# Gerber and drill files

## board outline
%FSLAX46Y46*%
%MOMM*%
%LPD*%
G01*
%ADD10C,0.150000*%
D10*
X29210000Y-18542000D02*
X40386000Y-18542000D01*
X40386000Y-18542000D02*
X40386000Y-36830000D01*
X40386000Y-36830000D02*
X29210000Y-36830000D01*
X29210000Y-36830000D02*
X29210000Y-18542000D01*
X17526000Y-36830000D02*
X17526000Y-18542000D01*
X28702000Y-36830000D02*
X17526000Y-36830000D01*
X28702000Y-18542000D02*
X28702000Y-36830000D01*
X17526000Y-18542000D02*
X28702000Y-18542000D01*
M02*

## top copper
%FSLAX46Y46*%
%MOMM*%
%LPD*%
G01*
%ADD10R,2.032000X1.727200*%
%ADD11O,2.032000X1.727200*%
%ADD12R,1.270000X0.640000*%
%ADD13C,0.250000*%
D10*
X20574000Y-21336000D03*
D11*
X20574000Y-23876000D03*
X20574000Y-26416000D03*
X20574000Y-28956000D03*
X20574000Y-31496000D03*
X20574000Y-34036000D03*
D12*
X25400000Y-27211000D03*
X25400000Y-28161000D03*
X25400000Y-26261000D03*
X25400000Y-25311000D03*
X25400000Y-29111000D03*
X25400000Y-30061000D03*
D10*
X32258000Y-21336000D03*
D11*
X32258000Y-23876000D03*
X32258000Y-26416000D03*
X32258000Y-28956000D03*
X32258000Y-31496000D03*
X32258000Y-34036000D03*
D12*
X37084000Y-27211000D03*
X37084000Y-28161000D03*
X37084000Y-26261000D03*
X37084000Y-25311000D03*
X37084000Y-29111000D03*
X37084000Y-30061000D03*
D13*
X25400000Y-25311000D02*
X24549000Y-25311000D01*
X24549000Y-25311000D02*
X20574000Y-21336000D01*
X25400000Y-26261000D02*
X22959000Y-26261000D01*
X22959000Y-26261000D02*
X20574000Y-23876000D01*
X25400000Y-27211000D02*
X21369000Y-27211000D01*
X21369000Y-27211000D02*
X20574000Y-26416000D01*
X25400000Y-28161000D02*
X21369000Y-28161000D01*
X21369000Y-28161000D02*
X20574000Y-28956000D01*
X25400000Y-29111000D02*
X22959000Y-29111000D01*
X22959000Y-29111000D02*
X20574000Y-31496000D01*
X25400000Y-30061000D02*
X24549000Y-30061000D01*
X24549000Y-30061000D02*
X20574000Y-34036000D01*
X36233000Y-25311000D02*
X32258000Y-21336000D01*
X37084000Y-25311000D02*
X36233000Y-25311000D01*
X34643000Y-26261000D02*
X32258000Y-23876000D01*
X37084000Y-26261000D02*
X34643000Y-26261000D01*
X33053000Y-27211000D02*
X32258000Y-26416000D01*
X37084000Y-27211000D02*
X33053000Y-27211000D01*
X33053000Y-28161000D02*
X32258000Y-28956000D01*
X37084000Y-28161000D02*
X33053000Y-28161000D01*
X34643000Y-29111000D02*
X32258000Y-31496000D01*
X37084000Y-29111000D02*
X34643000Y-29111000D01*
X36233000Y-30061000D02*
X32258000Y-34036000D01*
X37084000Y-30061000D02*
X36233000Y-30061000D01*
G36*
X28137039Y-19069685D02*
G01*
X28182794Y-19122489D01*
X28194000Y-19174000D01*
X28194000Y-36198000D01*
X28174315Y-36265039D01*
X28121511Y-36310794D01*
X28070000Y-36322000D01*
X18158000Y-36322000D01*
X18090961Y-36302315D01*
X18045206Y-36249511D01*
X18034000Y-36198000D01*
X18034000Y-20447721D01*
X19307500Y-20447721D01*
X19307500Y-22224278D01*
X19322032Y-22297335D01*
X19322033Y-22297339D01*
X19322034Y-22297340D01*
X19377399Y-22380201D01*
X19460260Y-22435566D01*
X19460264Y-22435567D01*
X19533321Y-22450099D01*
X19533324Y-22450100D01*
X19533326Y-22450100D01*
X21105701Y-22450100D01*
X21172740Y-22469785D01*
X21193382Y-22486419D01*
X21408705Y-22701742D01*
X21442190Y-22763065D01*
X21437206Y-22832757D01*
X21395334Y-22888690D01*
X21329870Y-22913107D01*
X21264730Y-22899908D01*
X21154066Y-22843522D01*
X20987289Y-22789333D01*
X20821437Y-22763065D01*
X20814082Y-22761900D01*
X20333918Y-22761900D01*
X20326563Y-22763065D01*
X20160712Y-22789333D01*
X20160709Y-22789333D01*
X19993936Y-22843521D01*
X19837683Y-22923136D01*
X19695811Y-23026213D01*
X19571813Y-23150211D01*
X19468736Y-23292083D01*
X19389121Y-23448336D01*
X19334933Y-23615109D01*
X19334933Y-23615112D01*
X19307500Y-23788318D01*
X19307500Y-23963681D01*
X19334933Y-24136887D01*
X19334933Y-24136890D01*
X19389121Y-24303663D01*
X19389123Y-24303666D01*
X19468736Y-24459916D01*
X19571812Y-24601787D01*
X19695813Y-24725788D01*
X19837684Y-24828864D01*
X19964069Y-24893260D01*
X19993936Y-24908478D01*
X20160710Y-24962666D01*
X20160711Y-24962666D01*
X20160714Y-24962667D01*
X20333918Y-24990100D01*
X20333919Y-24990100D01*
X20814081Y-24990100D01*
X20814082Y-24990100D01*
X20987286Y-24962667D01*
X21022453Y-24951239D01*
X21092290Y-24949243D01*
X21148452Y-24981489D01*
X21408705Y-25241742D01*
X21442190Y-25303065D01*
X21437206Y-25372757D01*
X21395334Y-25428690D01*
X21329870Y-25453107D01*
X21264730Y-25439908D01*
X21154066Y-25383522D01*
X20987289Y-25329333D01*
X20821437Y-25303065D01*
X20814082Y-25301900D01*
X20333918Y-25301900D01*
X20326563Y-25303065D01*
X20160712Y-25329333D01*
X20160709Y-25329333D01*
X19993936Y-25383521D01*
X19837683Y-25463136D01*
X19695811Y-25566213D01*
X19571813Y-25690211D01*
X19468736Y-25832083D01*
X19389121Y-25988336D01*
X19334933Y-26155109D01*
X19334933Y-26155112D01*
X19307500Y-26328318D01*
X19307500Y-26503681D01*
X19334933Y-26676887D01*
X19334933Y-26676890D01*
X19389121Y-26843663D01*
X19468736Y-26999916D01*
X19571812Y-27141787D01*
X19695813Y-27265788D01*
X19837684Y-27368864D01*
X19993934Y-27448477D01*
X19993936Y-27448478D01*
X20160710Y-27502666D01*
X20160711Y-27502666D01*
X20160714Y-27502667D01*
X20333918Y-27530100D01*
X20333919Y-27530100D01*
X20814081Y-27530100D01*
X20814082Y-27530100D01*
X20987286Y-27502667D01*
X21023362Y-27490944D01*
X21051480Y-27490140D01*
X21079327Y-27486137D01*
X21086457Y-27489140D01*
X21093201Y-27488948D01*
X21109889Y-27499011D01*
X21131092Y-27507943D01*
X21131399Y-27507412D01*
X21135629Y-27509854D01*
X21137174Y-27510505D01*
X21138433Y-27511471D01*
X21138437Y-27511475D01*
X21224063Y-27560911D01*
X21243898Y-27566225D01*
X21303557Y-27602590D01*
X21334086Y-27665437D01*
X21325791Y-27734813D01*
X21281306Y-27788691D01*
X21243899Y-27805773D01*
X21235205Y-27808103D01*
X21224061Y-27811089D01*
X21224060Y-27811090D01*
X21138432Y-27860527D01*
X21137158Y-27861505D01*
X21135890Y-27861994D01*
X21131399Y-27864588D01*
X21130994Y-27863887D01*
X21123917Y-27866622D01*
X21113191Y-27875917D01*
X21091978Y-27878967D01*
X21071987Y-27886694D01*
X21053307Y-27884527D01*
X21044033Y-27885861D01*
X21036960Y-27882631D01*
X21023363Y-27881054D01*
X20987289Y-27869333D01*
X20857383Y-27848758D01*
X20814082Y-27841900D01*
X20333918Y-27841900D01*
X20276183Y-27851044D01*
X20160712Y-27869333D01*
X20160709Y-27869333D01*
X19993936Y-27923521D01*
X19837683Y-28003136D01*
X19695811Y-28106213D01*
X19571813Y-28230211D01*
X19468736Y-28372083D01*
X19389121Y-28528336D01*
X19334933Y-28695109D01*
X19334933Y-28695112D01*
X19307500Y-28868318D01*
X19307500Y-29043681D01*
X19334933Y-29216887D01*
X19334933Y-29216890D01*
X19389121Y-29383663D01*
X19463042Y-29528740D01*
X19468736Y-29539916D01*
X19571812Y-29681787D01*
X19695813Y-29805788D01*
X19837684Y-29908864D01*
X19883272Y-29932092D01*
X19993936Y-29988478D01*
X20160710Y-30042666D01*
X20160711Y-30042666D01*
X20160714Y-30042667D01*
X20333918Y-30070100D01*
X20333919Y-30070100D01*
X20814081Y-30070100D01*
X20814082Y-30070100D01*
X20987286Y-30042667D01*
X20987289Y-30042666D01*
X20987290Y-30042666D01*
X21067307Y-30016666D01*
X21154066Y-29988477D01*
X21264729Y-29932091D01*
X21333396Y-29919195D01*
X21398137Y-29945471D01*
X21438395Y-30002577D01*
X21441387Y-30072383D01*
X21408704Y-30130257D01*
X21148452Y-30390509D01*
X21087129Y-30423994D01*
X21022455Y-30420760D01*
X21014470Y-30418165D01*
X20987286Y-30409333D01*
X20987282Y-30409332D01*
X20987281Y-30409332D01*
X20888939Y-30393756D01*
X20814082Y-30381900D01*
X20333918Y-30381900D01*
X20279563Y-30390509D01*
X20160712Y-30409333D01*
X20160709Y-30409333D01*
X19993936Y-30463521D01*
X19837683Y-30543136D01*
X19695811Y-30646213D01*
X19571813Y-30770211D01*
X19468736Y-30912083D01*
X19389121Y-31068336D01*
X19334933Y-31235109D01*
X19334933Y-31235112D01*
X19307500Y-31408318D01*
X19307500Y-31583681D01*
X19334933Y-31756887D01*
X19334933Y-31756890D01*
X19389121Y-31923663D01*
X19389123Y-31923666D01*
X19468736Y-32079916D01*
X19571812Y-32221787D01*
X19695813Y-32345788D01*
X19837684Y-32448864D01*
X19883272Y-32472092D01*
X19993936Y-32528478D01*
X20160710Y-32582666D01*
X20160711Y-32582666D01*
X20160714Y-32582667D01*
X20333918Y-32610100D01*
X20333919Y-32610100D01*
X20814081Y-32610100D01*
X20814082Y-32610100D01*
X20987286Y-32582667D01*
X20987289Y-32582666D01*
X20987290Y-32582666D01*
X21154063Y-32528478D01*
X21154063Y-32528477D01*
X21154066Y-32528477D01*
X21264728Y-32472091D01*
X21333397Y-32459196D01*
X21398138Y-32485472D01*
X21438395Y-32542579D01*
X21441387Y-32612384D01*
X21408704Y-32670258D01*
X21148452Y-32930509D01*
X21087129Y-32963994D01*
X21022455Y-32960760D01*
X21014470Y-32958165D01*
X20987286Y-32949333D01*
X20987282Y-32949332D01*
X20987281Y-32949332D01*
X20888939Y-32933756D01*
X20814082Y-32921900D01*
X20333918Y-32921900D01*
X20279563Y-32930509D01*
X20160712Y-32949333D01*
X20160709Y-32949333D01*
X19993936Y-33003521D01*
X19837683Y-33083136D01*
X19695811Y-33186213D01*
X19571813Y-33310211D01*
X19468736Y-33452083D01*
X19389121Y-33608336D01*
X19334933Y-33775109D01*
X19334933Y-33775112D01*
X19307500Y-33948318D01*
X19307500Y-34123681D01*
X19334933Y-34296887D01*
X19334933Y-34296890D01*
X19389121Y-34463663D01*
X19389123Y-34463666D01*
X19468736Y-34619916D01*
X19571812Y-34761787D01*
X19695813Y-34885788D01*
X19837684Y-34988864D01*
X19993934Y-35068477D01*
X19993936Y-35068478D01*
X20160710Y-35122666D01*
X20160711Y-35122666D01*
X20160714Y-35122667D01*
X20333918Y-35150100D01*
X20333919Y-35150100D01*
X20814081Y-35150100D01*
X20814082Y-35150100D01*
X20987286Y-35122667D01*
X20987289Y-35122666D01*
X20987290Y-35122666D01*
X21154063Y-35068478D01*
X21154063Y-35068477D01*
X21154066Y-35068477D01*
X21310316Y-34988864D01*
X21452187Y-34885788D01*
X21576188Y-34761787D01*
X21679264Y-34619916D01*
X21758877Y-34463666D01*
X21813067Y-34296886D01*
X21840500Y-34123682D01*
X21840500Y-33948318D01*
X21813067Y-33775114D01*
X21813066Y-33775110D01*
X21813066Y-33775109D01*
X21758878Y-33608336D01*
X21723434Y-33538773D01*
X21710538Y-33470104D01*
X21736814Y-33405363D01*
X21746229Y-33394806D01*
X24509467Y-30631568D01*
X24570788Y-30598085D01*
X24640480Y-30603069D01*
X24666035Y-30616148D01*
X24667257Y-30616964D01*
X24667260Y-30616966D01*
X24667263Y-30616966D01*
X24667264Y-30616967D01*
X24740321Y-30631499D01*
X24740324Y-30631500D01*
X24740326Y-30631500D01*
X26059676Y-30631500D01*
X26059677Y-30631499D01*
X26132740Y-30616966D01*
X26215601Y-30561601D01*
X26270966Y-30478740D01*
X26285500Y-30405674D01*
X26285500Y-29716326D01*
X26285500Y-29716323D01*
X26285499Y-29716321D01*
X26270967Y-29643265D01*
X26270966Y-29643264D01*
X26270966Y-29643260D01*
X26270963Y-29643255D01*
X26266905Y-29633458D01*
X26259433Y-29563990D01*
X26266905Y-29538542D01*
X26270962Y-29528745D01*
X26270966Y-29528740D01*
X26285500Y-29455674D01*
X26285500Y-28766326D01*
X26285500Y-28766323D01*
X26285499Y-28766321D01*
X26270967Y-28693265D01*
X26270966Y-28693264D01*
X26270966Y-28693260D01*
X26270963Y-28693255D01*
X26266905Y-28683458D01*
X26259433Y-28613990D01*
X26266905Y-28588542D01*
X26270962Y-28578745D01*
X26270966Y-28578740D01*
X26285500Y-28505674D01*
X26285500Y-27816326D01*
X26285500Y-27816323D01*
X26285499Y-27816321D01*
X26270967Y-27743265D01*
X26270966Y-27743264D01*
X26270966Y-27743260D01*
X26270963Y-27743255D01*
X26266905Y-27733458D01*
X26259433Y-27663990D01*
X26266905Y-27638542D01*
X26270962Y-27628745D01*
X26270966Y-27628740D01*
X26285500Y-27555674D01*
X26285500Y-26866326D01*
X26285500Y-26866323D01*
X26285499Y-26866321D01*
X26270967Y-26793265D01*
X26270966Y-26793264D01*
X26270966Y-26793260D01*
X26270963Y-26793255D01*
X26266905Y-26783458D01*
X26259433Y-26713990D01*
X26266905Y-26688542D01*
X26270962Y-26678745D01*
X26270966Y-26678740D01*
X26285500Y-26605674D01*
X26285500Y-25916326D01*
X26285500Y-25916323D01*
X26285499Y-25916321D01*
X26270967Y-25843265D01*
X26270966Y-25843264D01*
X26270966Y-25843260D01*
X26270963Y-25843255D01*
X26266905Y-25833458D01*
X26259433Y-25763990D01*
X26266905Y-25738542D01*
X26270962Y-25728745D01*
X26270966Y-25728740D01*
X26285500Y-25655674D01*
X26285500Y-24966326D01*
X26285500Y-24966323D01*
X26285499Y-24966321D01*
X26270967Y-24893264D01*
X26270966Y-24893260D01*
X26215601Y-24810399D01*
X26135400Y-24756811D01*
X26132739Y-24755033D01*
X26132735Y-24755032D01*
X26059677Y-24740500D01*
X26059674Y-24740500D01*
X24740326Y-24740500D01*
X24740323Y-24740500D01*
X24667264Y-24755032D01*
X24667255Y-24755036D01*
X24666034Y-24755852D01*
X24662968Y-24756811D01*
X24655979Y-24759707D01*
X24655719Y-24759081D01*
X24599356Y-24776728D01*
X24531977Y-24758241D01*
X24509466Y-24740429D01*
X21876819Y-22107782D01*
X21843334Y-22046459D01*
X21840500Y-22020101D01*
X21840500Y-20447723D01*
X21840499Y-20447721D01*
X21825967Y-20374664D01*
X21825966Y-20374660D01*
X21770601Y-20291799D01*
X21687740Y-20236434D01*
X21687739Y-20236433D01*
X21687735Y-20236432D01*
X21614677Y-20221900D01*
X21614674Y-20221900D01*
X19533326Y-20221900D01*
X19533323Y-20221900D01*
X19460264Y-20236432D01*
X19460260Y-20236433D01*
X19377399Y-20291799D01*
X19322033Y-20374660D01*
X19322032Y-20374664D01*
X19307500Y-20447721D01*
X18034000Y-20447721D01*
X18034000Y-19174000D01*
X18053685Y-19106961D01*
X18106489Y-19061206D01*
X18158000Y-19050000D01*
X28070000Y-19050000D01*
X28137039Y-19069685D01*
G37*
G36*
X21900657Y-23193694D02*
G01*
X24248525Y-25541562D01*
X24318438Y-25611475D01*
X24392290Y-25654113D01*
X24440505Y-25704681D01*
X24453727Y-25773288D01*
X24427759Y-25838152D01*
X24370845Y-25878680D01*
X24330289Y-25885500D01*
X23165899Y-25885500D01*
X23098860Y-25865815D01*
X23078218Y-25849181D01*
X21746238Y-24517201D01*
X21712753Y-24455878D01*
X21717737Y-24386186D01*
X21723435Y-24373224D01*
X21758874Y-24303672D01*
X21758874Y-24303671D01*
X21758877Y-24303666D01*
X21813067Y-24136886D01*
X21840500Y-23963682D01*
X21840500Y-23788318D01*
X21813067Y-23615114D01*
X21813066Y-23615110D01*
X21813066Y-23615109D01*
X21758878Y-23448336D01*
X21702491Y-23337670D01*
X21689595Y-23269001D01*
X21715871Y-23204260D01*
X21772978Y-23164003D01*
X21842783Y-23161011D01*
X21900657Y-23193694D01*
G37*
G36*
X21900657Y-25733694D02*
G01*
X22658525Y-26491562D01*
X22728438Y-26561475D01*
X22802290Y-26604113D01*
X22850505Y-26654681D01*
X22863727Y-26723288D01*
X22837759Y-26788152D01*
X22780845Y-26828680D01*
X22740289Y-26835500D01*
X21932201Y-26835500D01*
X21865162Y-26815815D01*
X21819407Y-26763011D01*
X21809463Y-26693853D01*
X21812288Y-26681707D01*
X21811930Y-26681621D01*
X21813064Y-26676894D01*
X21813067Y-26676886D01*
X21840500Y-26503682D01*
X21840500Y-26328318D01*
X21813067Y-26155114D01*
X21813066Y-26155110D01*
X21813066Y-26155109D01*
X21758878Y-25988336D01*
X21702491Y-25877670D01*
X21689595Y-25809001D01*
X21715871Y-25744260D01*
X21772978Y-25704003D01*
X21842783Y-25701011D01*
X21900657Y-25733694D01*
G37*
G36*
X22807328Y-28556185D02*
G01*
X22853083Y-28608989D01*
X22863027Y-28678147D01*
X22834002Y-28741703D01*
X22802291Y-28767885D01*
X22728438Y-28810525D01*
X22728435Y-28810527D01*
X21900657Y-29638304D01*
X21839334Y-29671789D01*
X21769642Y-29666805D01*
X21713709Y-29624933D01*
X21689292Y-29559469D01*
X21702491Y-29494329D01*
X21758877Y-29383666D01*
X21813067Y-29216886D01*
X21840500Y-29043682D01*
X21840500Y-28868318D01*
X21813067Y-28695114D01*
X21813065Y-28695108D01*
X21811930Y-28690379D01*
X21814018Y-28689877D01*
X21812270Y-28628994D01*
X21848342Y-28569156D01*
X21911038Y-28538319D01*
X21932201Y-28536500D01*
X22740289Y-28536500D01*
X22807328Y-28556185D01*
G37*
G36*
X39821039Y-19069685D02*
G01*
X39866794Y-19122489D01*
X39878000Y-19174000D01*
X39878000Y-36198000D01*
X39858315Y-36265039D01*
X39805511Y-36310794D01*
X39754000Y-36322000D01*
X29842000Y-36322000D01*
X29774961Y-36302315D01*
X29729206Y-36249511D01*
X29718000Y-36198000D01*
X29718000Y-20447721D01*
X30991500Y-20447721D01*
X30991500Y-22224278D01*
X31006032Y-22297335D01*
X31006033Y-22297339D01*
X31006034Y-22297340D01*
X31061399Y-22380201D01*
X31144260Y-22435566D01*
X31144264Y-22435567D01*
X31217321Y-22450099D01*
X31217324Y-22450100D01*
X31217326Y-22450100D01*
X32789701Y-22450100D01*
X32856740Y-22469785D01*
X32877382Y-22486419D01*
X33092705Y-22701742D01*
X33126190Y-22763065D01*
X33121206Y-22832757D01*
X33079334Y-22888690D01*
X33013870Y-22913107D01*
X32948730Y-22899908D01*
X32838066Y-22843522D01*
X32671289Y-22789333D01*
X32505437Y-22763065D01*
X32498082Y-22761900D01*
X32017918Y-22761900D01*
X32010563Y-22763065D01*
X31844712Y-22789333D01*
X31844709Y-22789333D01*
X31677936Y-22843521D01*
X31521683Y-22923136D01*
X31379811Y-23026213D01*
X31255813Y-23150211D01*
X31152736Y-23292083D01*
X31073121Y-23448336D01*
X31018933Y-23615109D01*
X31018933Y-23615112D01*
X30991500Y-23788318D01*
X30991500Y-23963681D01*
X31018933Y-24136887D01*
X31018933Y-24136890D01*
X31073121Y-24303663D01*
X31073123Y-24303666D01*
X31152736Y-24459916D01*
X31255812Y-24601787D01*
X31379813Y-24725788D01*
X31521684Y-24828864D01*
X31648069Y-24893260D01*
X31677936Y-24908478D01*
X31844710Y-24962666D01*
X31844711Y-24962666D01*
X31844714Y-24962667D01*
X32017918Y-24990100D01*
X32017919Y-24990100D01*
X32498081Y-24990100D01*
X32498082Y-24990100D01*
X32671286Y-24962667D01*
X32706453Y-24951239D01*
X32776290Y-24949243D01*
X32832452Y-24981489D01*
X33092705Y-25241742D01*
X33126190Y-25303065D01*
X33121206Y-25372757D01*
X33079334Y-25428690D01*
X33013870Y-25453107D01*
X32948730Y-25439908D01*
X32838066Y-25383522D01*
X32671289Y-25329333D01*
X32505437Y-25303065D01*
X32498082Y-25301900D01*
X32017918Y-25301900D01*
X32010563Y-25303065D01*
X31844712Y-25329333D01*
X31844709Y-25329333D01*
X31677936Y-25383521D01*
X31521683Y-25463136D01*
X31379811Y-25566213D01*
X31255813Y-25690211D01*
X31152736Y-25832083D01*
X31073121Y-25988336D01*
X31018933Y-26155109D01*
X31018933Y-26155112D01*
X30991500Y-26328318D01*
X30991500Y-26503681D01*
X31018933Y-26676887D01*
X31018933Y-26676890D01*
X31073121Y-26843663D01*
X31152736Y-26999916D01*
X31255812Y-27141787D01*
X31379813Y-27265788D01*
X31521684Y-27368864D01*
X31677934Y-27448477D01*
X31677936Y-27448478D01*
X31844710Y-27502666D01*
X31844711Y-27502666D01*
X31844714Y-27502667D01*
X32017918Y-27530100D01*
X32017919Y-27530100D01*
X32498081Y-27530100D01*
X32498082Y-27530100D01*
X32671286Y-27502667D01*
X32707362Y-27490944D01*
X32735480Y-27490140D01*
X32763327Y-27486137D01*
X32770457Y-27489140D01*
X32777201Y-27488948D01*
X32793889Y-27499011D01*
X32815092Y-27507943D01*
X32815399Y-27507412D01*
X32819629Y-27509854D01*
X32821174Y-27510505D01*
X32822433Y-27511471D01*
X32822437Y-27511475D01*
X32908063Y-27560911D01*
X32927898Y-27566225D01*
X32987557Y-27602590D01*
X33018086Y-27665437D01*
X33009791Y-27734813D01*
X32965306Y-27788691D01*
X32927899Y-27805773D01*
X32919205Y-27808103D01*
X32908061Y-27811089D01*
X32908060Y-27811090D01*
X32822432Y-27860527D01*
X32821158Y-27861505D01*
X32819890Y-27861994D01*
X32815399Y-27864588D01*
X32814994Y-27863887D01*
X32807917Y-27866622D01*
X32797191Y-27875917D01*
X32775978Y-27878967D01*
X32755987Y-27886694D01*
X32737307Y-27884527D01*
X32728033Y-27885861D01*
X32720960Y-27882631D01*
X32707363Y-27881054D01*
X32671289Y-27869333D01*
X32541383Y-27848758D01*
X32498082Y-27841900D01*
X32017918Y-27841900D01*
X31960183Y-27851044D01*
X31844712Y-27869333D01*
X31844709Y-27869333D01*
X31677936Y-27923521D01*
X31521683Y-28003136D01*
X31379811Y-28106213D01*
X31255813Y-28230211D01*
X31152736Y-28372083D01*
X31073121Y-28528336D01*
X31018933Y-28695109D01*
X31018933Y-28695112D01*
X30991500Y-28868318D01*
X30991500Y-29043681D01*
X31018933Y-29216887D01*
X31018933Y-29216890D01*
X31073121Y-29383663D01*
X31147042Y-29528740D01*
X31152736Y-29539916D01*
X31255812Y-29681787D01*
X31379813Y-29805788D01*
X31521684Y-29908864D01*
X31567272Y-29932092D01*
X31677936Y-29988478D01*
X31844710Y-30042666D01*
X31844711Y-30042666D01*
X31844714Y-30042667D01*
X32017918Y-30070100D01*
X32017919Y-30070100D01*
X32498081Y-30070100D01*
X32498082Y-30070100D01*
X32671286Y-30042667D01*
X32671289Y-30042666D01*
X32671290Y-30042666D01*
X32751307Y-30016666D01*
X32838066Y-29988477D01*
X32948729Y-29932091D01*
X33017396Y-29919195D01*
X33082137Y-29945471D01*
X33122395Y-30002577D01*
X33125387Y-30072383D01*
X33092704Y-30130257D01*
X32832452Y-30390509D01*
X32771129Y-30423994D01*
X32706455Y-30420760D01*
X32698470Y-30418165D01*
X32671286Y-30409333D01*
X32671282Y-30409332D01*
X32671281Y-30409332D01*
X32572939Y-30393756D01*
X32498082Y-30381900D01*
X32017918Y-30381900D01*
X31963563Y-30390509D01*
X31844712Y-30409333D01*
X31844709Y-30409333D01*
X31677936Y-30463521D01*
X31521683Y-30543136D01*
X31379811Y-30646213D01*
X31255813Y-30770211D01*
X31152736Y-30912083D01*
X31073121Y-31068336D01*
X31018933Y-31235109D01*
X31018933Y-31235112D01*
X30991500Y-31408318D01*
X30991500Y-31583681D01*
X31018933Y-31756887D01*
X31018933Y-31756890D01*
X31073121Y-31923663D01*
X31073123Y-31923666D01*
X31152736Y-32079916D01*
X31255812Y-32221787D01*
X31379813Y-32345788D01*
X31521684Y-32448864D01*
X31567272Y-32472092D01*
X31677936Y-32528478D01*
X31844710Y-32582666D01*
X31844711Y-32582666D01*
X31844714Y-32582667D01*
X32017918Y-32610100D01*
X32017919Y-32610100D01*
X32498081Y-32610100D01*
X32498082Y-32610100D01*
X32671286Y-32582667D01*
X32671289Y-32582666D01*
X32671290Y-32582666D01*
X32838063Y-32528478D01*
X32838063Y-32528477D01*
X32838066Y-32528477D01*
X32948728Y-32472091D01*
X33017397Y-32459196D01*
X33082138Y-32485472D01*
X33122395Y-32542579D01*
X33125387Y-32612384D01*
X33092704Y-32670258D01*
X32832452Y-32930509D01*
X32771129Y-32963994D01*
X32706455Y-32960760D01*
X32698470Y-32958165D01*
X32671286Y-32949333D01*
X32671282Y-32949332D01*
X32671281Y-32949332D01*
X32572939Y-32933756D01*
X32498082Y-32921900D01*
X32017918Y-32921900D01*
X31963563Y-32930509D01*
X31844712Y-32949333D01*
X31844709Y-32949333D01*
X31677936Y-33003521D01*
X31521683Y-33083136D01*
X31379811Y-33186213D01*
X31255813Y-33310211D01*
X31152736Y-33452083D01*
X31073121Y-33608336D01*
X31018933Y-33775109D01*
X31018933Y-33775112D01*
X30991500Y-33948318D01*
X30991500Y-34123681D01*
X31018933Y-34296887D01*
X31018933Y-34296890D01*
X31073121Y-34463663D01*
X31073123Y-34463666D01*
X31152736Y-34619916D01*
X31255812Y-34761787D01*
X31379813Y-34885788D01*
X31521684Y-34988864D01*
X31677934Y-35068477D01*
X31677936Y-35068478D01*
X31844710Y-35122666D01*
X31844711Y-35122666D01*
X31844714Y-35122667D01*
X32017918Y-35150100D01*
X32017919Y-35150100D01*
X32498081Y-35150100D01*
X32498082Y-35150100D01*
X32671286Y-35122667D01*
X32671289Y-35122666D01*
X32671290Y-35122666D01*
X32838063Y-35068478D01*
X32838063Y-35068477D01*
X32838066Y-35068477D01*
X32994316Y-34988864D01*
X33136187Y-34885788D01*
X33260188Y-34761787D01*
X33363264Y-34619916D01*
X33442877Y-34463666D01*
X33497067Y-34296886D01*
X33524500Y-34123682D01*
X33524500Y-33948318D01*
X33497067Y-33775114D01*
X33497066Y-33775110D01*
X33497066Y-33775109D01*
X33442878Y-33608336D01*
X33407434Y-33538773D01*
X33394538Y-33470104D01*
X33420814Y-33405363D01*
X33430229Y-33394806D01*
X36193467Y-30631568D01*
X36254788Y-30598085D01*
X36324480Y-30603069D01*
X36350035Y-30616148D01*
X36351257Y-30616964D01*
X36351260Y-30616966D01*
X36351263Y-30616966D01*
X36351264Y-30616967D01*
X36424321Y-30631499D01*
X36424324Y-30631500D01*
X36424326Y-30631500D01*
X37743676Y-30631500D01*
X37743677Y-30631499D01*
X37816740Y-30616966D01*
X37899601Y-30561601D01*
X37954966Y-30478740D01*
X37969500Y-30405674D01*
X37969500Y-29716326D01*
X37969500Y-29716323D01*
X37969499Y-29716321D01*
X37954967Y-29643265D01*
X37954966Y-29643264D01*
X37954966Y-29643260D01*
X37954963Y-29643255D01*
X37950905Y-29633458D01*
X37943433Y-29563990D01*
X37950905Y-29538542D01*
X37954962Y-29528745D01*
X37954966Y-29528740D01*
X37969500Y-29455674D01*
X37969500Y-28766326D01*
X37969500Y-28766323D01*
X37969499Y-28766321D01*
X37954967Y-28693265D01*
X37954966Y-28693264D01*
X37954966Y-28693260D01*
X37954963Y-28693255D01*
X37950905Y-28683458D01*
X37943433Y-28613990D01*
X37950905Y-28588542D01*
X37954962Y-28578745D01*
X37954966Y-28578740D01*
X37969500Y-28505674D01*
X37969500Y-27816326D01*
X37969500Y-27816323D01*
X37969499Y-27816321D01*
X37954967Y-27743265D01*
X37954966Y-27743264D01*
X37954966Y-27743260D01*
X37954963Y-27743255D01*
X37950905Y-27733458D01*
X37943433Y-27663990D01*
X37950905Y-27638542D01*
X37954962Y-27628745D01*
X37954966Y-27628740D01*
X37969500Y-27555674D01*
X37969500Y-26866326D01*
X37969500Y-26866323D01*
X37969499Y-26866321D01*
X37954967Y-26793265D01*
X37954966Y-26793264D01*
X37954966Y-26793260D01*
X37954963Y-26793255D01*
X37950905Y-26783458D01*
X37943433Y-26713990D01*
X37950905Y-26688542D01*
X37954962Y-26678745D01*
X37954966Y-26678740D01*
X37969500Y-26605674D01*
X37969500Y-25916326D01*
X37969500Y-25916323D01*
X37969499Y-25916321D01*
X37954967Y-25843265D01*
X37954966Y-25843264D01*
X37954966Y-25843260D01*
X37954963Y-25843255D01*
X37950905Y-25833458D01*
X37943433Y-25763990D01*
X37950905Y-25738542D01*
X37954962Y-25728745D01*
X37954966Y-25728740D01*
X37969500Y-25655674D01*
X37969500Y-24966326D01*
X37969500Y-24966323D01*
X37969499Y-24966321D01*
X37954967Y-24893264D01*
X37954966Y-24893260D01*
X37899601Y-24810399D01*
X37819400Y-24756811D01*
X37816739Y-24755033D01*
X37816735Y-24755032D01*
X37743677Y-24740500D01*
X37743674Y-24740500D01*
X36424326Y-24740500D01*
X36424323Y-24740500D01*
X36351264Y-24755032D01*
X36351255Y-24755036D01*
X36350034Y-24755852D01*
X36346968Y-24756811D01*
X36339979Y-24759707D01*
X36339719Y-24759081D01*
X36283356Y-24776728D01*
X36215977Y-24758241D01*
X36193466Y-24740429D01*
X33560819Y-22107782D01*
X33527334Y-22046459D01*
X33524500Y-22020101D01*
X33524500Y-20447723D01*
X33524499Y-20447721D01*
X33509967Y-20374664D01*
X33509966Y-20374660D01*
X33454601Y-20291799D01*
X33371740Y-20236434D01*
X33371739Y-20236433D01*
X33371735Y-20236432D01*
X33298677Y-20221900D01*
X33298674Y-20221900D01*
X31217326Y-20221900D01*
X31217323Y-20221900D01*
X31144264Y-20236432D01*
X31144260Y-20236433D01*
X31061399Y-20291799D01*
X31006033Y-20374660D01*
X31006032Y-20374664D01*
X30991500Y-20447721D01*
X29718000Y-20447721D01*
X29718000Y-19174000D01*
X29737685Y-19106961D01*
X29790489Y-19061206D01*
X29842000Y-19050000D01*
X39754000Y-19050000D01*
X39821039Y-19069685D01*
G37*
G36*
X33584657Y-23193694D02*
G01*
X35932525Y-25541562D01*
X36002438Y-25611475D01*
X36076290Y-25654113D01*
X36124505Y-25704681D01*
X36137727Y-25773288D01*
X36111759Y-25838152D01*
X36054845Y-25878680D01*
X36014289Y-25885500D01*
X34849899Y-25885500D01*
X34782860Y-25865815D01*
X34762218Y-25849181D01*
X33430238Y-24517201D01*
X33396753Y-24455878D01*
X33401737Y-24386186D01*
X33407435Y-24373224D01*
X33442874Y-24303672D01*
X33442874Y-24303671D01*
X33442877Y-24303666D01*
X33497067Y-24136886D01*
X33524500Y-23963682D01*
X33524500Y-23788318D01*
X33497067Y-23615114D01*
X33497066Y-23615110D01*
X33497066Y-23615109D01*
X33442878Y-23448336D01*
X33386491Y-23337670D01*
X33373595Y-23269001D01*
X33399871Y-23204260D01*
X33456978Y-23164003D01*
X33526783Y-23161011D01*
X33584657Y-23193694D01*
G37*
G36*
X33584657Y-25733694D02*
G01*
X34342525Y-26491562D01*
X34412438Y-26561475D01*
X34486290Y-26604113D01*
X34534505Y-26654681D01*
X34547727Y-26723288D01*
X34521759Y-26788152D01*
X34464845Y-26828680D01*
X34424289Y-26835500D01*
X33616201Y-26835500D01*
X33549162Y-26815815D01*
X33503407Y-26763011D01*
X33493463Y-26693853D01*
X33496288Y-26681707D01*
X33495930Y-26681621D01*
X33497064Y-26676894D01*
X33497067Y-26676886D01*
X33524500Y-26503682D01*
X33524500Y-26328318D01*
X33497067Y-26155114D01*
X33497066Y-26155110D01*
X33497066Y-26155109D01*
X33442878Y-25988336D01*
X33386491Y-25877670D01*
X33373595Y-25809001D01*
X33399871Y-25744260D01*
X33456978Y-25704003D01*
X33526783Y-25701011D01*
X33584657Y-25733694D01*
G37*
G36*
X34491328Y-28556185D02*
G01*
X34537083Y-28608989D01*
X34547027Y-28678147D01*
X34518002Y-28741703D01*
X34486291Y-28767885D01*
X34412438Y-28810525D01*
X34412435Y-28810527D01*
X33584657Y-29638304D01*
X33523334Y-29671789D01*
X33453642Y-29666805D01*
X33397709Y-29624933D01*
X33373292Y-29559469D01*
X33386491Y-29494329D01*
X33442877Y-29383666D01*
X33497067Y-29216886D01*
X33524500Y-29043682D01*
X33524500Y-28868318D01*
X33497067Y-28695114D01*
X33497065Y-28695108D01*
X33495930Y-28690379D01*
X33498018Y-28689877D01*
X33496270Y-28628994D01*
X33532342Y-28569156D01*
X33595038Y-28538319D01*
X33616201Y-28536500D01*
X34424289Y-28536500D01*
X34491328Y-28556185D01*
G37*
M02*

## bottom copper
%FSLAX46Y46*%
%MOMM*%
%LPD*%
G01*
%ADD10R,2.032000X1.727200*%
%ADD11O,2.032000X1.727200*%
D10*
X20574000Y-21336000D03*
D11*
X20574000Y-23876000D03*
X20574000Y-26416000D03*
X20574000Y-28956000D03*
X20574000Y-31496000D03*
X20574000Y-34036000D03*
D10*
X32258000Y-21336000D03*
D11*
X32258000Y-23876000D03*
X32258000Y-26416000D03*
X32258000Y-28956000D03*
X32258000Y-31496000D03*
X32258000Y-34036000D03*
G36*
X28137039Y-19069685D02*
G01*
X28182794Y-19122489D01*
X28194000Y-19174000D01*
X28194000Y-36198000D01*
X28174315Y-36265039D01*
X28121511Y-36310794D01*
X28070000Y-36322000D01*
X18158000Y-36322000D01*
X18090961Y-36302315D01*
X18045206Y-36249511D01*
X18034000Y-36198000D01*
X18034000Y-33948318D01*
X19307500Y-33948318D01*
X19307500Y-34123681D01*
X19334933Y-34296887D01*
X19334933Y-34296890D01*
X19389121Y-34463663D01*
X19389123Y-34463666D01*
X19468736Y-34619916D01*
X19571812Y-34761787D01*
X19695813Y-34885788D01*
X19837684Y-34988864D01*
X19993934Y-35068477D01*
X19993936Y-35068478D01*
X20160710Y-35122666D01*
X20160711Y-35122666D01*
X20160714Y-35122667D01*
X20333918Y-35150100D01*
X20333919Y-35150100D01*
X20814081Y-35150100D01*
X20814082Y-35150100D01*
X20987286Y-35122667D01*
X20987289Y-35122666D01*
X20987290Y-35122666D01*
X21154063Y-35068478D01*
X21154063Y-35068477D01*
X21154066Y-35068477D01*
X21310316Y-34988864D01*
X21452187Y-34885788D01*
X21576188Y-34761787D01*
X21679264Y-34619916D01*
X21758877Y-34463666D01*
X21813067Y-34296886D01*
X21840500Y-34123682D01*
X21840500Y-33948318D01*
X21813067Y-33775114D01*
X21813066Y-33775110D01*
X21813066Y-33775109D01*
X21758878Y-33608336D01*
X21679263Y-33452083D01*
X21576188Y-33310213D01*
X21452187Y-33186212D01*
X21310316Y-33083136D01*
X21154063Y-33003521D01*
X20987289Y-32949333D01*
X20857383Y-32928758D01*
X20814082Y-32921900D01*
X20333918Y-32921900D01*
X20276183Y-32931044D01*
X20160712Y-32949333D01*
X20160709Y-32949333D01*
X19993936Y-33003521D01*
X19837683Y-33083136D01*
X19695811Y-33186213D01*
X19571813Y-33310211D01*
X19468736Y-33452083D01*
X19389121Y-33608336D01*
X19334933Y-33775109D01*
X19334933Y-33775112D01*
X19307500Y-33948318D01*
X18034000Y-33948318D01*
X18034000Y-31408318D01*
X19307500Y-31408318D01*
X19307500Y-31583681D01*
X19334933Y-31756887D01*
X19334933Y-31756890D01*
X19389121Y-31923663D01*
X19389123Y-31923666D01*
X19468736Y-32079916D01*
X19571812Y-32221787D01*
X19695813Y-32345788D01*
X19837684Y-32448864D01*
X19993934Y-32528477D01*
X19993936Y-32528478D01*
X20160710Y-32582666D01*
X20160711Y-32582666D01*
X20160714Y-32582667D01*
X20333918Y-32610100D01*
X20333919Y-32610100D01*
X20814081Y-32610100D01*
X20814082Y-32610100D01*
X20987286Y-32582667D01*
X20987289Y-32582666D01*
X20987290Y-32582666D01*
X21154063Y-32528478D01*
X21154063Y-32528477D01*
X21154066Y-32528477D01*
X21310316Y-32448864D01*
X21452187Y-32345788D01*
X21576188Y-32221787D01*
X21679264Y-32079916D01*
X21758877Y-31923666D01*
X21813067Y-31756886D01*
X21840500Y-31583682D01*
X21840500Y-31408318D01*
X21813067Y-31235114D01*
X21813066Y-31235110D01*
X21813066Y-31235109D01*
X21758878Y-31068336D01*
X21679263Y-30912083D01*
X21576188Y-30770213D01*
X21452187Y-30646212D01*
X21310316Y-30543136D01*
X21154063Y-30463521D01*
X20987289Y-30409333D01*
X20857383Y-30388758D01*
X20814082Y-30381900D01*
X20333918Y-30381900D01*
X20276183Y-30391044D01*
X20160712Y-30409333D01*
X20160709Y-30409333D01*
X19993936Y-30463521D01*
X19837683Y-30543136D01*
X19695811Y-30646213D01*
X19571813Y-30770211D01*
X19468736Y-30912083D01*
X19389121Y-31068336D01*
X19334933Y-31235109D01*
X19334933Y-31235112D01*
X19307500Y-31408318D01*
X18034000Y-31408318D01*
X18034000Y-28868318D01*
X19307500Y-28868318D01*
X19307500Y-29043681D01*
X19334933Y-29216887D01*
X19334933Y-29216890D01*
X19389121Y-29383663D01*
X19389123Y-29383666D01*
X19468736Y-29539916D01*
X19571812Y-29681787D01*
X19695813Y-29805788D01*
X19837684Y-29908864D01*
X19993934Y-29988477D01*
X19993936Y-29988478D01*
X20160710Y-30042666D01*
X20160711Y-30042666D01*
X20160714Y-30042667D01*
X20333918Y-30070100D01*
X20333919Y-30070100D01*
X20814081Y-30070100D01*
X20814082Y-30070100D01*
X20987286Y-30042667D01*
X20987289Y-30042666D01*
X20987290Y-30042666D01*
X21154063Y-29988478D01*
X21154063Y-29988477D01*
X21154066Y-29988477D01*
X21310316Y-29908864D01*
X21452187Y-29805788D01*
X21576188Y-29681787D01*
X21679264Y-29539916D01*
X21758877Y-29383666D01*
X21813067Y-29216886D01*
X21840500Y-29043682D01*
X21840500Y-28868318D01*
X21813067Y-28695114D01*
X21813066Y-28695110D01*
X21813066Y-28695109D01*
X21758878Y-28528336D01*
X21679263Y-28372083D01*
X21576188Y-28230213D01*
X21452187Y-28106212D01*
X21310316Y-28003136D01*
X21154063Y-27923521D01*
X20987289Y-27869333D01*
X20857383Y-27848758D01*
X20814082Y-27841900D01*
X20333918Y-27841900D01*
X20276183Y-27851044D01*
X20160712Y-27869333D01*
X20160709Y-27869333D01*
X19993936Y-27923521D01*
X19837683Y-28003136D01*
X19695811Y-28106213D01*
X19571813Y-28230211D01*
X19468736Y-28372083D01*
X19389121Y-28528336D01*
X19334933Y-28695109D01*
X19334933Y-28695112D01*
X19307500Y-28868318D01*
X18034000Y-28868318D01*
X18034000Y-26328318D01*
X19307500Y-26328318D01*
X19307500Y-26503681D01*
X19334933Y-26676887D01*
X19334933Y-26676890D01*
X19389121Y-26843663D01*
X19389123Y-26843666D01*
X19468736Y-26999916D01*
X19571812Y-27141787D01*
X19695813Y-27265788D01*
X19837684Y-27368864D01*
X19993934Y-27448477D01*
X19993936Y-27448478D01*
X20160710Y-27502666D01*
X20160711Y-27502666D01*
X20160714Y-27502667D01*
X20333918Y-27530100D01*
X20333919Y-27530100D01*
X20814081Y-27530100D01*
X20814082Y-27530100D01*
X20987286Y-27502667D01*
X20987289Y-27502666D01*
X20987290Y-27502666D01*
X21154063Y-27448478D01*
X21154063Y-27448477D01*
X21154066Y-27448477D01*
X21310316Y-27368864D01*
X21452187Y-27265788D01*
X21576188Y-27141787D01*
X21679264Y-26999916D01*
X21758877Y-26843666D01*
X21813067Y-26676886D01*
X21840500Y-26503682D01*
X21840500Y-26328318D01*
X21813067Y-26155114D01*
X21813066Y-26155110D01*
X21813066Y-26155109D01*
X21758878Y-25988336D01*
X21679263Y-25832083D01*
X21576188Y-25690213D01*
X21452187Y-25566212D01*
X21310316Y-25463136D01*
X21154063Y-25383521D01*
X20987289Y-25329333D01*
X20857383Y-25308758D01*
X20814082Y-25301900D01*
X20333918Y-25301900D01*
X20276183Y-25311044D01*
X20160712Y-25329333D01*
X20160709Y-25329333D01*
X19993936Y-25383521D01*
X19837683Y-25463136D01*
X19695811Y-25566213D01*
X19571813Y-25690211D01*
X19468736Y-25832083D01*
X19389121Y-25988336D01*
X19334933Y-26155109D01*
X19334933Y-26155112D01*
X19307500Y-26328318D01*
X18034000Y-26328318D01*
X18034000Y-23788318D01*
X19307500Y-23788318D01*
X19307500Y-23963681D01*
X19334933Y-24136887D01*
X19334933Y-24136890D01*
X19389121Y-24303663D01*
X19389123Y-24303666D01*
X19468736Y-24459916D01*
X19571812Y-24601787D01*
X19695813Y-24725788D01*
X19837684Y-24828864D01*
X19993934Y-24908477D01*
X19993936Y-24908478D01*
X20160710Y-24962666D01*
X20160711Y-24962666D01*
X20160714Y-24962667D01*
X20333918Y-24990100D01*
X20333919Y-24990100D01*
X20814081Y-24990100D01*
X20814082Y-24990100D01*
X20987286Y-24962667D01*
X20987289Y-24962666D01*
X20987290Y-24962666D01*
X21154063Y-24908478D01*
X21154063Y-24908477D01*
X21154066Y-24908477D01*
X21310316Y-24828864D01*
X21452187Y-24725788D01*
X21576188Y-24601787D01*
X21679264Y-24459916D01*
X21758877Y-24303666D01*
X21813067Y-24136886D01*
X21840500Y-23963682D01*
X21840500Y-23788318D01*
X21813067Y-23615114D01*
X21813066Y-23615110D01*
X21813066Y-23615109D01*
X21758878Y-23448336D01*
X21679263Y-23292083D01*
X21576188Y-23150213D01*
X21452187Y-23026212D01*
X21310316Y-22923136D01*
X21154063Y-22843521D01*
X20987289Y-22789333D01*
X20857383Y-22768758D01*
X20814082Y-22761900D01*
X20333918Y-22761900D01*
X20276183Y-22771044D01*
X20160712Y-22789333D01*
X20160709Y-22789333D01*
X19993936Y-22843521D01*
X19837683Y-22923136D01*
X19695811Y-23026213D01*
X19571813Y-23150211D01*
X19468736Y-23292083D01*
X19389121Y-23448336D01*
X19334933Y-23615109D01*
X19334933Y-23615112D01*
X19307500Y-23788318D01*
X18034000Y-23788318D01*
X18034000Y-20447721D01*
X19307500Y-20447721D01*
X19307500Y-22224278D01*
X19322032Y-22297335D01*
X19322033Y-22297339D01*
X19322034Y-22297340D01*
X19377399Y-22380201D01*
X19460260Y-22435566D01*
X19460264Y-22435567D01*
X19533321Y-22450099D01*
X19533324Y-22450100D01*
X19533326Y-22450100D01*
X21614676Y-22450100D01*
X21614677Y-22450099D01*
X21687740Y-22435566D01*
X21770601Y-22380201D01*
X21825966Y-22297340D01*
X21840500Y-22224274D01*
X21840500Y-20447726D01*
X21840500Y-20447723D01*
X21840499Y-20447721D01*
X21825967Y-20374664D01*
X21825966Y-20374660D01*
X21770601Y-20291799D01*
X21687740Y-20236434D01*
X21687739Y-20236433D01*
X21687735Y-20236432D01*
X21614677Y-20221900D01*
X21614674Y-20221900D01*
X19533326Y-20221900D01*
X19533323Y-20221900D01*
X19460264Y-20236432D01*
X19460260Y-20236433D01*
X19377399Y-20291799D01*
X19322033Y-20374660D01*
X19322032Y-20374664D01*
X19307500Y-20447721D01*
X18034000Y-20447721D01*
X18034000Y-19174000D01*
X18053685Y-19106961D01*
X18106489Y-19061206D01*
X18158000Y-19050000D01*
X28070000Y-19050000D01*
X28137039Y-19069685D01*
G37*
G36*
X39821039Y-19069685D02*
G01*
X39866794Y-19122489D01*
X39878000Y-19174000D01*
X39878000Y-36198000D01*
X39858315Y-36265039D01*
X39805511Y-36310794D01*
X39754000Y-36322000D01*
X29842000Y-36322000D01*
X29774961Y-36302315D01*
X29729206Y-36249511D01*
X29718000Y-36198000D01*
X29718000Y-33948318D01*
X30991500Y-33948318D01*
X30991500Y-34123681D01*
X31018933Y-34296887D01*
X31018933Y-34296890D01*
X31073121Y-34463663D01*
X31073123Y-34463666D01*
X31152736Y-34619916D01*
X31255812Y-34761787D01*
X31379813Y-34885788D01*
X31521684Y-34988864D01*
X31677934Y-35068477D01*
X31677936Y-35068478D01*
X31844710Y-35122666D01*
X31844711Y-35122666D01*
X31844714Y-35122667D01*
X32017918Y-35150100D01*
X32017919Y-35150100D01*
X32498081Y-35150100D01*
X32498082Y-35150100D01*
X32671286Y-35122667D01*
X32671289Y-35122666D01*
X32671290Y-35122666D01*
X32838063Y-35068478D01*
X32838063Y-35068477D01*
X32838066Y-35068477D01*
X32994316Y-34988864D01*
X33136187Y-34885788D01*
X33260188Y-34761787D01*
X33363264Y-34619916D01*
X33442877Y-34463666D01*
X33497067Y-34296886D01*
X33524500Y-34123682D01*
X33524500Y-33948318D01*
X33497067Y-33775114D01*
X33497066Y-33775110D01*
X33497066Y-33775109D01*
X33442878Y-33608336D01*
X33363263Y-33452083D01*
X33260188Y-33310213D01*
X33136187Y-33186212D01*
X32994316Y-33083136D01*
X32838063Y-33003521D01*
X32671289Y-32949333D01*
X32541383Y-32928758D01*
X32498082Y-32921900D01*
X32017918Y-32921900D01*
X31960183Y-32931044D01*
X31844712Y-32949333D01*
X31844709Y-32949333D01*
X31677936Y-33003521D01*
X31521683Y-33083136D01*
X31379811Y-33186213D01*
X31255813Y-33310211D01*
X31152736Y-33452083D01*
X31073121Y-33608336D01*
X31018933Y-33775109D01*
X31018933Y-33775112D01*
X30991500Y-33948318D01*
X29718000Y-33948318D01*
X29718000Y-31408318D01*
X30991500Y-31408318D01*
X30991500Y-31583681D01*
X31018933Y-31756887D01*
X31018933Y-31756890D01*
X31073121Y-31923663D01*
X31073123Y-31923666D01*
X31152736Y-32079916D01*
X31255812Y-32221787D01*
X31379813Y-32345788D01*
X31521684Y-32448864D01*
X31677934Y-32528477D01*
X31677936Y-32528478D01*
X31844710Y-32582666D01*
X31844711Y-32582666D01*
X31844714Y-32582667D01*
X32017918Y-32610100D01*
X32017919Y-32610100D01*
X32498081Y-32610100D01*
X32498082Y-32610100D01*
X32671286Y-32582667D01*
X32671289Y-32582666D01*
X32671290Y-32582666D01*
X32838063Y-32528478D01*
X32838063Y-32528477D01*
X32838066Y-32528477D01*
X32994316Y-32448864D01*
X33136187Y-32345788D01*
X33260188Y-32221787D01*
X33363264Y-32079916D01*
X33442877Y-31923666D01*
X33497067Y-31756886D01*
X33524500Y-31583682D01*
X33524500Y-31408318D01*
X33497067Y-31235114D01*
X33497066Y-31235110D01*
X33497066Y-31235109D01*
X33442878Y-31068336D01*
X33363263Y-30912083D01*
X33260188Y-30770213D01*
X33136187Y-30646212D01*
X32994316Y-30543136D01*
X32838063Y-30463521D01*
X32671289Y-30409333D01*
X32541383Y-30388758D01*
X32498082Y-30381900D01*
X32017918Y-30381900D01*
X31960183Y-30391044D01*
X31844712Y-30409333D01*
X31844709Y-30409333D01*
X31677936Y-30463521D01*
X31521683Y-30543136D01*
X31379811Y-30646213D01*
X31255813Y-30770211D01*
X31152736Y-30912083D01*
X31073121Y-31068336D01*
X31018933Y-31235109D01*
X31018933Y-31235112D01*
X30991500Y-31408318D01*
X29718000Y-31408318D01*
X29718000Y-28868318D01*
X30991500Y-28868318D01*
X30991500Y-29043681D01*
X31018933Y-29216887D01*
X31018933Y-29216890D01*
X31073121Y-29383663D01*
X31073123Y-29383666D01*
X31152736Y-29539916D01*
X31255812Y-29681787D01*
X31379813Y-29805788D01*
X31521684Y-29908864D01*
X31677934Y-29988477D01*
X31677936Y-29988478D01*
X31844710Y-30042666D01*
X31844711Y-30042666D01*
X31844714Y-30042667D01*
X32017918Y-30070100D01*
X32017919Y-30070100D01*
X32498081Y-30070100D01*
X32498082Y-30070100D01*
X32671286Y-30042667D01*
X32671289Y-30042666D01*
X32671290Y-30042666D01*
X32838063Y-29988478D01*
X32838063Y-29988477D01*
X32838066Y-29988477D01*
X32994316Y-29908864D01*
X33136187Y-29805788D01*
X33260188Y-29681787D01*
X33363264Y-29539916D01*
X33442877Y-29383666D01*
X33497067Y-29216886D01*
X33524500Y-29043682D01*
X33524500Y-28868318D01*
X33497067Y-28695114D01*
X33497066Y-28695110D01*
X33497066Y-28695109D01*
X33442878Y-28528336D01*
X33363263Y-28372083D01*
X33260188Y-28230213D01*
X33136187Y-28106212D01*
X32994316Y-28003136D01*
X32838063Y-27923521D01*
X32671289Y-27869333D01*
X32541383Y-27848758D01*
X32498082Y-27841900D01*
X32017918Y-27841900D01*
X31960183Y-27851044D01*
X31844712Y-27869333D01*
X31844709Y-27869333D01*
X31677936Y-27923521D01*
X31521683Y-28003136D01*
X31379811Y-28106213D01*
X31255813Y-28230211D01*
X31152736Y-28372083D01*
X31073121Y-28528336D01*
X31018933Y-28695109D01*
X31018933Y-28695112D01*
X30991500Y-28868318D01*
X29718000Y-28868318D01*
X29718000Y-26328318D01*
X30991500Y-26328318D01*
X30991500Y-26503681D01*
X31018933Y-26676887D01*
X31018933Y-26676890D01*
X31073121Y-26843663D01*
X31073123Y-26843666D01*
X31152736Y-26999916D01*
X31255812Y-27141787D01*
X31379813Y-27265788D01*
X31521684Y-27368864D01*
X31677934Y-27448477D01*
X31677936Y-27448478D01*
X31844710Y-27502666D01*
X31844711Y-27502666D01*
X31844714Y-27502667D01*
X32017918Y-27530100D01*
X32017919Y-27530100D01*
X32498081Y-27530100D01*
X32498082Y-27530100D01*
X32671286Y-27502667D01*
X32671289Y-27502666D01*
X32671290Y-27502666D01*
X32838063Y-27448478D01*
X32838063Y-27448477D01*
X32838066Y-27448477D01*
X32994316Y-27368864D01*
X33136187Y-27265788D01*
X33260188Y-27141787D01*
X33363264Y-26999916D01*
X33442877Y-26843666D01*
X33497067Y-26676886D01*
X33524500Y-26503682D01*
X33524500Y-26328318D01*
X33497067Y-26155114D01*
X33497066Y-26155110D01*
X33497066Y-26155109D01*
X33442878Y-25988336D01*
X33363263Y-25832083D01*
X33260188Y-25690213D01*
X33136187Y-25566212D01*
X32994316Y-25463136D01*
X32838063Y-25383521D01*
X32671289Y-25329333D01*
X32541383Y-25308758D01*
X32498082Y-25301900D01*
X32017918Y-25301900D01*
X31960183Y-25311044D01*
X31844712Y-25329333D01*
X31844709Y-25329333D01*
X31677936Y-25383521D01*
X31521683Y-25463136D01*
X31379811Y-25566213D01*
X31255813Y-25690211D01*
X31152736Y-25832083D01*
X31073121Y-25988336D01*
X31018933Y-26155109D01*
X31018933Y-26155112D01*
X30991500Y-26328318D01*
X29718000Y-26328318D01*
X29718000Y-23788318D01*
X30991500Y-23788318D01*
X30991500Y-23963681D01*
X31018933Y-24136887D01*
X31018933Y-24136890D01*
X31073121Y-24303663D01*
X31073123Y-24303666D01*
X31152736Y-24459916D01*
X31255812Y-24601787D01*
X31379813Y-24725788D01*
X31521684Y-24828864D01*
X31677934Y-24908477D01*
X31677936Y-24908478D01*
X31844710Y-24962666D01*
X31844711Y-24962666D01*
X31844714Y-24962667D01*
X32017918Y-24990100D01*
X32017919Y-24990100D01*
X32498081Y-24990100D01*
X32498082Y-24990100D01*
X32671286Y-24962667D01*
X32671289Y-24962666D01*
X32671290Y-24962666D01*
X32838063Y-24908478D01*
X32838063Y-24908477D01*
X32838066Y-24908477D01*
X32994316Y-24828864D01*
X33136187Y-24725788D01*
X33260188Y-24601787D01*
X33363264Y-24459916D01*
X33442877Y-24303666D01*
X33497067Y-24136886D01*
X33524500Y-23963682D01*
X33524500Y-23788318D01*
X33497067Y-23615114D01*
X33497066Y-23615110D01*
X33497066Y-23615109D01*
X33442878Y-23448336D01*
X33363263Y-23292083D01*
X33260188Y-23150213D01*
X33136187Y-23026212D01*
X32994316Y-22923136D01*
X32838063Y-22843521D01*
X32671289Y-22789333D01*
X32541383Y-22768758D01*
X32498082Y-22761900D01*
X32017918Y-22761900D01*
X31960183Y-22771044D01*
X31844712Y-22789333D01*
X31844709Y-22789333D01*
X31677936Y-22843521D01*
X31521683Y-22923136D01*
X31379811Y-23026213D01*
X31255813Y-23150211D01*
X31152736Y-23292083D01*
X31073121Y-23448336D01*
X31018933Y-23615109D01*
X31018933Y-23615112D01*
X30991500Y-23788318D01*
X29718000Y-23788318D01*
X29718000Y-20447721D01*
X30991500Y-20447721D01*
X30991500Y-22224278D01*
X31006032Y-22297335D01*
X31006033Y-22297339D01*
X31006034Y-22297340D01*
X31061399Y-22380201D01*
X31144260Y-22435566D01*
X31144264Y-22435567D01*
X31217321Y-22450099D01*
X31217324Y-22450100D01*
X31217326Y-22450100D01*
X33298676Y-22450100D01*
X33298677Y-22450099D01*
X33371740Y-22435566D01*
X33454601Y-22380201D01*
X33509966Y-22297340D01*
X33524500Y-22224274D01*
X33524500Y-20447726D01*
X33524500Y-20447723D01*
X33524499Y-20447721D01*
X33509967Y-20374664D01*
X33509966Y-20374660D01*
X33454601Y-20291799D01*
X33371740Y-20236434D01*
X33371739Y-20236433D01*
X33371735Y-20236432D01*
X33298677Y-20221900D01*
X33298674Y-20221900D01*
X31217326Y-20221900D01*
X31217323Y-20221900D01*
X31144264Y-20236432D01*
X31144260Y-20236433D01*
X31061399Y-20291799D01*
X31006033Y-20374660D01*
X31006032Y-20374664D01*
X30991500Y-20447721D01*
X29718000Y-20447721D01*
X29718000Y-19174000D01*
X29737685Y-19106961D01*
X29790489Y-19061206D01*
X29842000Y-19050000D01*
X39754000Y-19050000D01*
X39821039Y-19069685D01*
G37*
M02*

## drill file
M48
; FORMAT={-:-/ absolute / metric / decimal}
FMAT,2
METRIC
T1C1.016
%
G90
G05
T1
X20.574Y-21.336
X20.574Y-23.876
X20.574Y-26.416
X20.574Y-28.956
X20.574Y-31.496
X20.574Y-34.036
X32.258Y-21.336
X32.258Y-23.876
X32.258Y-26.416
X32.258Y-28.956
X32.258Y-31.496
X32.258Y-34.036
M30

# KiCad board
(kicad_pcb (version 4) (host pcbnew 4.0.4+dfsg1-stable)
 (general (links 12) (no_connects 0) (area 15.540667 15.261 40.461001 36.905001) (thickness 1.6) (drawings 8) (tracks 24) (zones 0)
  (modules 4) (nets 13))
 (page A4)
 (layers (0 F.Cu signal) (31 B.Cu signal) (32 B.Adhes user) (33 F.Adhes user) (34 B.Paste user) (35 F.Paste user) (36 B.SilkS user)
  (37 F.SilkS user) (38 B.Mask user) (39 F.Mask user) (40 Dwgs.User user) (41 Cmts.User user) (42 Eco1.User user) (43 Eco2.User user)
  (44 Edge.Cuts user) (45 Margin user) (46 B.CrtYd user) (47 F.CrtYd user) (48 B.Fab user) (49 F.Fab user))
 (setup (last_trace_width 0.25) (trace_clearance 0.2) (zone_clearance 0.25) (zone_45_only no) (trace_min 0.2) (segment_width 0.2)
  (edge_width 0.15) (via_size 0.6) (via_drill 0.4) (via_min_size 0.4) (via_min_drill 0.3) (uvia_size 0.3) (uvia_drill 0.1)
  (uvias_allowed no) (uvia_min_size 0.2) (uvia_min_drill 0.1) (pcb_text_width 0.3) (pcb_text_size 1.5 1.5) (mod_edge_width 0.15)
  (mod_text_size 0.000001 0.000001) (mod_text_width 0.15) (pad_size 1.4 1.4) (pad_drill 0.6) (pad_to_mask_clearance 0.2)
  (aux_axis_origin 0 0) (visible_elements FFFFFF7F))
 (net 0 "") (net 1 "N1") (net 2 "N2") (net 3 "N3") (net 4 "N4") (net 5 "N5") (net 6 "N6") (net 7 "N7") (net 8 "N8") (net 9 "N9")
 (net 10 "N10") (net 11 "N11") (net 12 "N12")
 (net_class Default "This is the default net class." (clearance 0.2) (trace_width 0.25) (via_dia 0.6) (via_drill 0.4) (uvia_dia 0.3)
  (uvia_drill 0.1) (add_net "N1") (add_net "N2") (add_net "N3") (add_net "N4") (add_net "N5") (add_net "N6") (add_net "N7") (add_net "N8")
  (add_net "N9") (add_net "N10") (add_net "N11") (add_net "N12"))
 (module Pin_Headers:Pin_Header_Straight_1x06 (layer F.Cu) (at 20.574 21.336)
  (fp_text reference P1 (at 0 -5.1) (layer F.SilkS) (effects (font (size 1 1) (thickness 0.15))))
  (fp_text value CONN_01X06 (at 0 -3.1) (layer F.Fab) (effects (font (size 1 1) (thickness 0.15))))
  (pad 1 thru_hole rect (at 0 0) (size 2.032 1.7272) (drill 1.016) (layers *.Cu *.Mask F.SilkS) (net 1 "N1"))
  (pad 2 thru_hole oval (at 0 2.54) (size 2.032 1.7272) (drill 1.016) (layers *.Cu *.Mask F.SilkS) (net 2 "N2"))
  (pad 3 thru_hole oval (at 0 5.08) (size 2.032 1.7272) (drill 1.016) (layers *.Cu *.Mask F.SilkS) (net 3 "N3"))
  (pad 4 thru_hole oval (at 0 7.62) (size 2.032 1.7272) (drill 1.016) (layers *.Cu *.Mask F.SilkS) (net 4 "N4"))
  (pad 5 thru_hole oval (at 0 10.16) (size 2.032 1.7272) (drill 1.016) (layers *.Cu *.Mask F.SilkS) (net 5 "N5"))
  (pad 6 thru_hole oval (at 0 12.7) (size 2.032 1.7272) (drill 1.016) (layers *.Cu *.Mask F.SilkS) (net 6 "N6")))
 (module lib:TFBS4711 (layer F.Cu) (at 25.4 27.686 90)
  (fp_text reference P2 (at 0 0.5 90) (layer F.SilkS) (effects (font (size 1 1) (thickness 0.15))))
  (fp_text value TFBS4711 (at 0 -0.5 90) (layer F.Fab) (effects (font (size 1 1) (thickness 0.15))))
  (pad 4 smd rect (at 0.475 0 90) (size 0.64 1.27) (layers F.Cu F.Paste F.Mask) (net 3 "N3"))
  (pad 3 smd rect (at -0.475 0 90) (size 0.64 1.27) (layers F.Cu F.Paste F.Mask) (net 4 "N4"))
  (pad 5 smd rect (at 1.425 0 90) (size 0.64 1.27) (layers F.Cu F.Paste F.Mask) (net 2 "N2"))
  (pad 6 smd rect (at 2.375 0 90) (size 0.64 1.27) (layers F.Cu F.Paste F.Mask) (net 1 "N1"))
  (pad 2 smd rect (at -1.425 0 90) (size 0.64 1.27) (layers F.Cu F.Paste F.Mask) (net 5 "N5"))
  (pad 1 smd rect (at -2.375 0 90) (size 0.64 1.27) (layers F.Cu F.Paste F.Mask) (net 6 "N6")))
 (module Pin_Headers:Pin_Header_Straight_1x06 (layer F.Cu) (at 32.258 21.336)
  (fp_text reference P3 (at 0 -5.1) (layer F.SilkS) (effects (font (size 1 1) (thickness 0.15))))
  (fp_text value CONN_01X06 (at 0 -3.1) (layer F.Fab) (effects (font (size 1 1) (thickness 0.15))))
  (pad 1 thru_hole rect (at 0 0) (size 2.032 1.7272) (drill 1.016) (layers *.Cu *.Mask F.SilkS) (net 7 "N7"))
  (pad 2 thru_hole oval (at 0 2.54) (size 2.032 1.7272) (drill 1.016) (layers *.Cu *.Mask F.SilkS) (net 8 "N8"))
  (pad 3 thru_hole oval (at 0 5.08) (size 2.032 1.7272) (drill 1.016) (layers *.Cu *.Mask F.SilkS) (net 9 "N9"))
  (pad 4 thru_hole oval (at 0 7.62) (size 2.032 1.7272) (drill 1.016) (layers *.Cu *.Mask F.SilkS) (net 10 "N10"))
  (pad 5 thru_hole oval (at 0 10.16) (size 2.032 1.7272) (drill 1.016) (layers *.Cu *.Mask F.SilkS) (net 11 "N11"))
  (pad 6 thru_hole oval (at 0 12.7) (size 2.032 1.7272) (drill 1.016) (layers *.Cu *.Mask F.SilkS) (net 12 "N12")))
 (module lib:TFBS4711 (layer F.Cu) (at 37.084 27.686 90)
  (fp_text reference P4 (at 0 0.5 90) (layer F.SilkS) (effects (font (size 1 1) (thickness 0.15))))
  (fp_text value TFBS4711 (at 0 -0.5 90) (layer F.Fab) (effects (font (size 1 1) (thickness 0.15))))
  (pad 4 smd rect (at 0.475 0 90) (size 0.64 1.27) (layers F.Cu F.Paste F.Mask) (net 9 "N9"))
  (pad 3 smd rect (at -0.475 0 90) (size 0.64 1.27) (layers F.Cu F.Paste F.Mask) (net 10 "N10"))
  (pad 5 smd rect (at 1.425 0 90) (size 0.64 1.27) (layers F.Cu F.Paste F.Mask) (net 8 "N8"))
  (pad 6 smd rect (at 2.375 0 90) (size 0.64 1.27) (layers F.Cu F.Paste F.Mask) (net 7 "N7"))
  (pad 2 smd rect (at -1.425 0 90) (size 0.64 1.27) (layers F.Cu F.Paste F.Mask) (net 11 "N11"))
  (pad 1 smd rect (at -2.375 0 90) (size 0.64 1.27) (layers F.Cu F.Paste F.Mask) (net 12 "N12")))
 (gr_line (start 29.21 18.542) (end 40.386 18.542) (angle 90) (layer Edge.Cuts) (width 0.15))
 (gr_line (start 40.386 18.542) (end 40.386 36.83) (angle 90) (layer Edge.Cuts) (width 0.15))
 (gr_line (start 40.386 36.83) (end 29.21 36.83) (angle 90) (layer Edge.Cuts) (width 0.15))
 (gr_line (start 29.21 36.83) (end 29.21 18.542) (angle 90) (layer Edge.Cuts) (width 0.15))
 (gr_line (start 17.526 36.83) (end 17.526 18.542) (angle 90) (layer Edge.Cuts) (width 0.15))
 (gr_line (start 28.702 36.83) (end 17.526 36.83) (angle 90) (layer Edge.Cuts) (width 0.15))
 (gr_line (start 28.702 18.542) (end 28.702 36.83) (angle 90) (layer Edge.Cuts) (width 0.15))
 (gr_line (start 17.526 18.542) (end 28.702 18.542) (angle 90) (layer Edge.Cuts) (width 0.15))
 (segment (start 25.4 25.311) (end 24.549 25.311) (width 0.25) (layer F.Cu) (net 1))
 (segment (start 24.549 25.311) (end 20.574 21.336) (width 0.25) (layer F.Cu) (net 1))
 (segment (start 25.4 26.261) (end 22.959 26.261) (width 0.25) (layer F.Cu) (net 2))
 (segment (start 22.959 26.261) (end 20.574 23.876) (width 0.25) (layer F.Cu) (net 2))
 (segment (start 25.4 27.211) (end 21.369 27.211) (width 0.25) (layer F.Cu) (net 3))
 (segment (start 21.369 27.211) (end 20.574 26.416) (width 0.25) (layer F.Cu) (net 3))
 (segment (start 25.4 28.161) (end 21.369 28.161) (width 0.25) (layer F.Cu) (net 4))
 (segment (start 21.369 28.161) (end 20.574 28.956) (width 0.25) (layer F.Cu) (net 4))
 (segment (start 25.4 29.111) (end 22.959 29.111) (width 0.25) (layer F.Cu) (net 5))
 (segment (start 22.959 29.111) (end 20.574 31.496) (width 0.25) (layer F.Cu) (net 5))
 (segment (start 25.4 30.061) (end 24.549 30.061) (width 0.25) (layer F.Cu) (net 6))
 (segment (start 24.549 30.061) (end 20.574 34.036) (width 0.25) (layer F.Cu) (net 6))
 (segment (start 36.233 25.311) (end 32.258 21.336) (width 0.25) (layer F.Cu) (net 7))
 (segment (start 37.084 25.311) (end 36.233 25.311) (width 0.25) (layer F.Cu) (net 7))
 (segment (start 34.643 26.261) (end 32.258 23.876) (width 0.25) (layer F.Cu) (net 8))
 (segment (start 37.084 26.261) (end 34.643 26.261) (width 0.25) (layer F.Cu) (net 8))
 (segment (start 33.053 27.211) (end 32.258 26.416) (width 0.25) (layer F.Cu) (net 9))
 (segment (start 37.084 27.211) (end 33.053 27.211) (width 0.25) (layer F.Cu) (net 9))
 (segment (start 33.053 28.161) (end 32.258 28.956) (width 0.25) (layer F.Cu) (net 10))
 (segment (start 37.084 28.161) (end 33.053 28.161) (width 0.25) (layer F.Cu) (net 10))
 (segment (start 34.643 29.111) (end 32.258 31.496) (width 0.25) (layer F.Cu) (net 11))
 (segment (start 37.084 29.111) (end 34.643 29.111) (width 0.25) (layer F.Cu) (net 11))
 (segment (start 36.233 30.061) (end 32.258 34.036) (width 0.25) (layer F.Cu) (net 12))
 (segment (start 37.084 30.061) (end 36.233 30.061) (width 0.25) (layer F.Cu) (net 12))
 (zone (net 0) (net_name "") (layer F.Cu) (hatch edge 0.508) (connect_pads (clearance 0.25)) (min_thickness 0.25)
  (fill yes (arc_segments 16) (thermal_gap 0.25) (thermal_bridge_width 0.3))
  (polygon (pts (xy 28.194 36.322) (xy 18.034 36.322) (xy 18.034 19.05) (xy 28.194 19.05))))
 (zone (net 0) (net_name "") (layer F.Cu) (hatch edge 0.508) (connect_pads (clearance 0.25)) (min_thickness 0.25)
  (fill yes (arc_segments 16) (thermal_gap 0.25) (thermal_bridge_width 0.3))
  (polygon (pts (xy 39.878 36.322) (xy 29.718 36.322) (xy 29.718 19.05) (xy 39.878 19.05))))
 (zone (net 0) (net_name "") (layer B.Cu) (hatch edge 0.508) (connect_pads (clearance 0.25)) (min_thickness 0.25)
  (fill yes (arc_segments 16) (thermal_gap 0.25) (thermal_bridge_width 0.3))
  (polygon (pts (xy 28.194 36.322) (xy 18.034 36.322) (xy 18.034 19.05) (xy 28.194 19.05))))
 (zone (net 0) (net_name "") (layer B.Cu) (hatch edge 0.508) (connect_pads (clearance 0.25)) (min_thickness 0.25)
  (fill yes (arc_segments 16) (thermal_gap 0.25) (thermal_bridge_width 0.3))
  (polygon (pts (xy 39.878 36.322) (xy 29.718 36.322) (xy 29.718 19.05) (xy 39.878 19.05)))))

